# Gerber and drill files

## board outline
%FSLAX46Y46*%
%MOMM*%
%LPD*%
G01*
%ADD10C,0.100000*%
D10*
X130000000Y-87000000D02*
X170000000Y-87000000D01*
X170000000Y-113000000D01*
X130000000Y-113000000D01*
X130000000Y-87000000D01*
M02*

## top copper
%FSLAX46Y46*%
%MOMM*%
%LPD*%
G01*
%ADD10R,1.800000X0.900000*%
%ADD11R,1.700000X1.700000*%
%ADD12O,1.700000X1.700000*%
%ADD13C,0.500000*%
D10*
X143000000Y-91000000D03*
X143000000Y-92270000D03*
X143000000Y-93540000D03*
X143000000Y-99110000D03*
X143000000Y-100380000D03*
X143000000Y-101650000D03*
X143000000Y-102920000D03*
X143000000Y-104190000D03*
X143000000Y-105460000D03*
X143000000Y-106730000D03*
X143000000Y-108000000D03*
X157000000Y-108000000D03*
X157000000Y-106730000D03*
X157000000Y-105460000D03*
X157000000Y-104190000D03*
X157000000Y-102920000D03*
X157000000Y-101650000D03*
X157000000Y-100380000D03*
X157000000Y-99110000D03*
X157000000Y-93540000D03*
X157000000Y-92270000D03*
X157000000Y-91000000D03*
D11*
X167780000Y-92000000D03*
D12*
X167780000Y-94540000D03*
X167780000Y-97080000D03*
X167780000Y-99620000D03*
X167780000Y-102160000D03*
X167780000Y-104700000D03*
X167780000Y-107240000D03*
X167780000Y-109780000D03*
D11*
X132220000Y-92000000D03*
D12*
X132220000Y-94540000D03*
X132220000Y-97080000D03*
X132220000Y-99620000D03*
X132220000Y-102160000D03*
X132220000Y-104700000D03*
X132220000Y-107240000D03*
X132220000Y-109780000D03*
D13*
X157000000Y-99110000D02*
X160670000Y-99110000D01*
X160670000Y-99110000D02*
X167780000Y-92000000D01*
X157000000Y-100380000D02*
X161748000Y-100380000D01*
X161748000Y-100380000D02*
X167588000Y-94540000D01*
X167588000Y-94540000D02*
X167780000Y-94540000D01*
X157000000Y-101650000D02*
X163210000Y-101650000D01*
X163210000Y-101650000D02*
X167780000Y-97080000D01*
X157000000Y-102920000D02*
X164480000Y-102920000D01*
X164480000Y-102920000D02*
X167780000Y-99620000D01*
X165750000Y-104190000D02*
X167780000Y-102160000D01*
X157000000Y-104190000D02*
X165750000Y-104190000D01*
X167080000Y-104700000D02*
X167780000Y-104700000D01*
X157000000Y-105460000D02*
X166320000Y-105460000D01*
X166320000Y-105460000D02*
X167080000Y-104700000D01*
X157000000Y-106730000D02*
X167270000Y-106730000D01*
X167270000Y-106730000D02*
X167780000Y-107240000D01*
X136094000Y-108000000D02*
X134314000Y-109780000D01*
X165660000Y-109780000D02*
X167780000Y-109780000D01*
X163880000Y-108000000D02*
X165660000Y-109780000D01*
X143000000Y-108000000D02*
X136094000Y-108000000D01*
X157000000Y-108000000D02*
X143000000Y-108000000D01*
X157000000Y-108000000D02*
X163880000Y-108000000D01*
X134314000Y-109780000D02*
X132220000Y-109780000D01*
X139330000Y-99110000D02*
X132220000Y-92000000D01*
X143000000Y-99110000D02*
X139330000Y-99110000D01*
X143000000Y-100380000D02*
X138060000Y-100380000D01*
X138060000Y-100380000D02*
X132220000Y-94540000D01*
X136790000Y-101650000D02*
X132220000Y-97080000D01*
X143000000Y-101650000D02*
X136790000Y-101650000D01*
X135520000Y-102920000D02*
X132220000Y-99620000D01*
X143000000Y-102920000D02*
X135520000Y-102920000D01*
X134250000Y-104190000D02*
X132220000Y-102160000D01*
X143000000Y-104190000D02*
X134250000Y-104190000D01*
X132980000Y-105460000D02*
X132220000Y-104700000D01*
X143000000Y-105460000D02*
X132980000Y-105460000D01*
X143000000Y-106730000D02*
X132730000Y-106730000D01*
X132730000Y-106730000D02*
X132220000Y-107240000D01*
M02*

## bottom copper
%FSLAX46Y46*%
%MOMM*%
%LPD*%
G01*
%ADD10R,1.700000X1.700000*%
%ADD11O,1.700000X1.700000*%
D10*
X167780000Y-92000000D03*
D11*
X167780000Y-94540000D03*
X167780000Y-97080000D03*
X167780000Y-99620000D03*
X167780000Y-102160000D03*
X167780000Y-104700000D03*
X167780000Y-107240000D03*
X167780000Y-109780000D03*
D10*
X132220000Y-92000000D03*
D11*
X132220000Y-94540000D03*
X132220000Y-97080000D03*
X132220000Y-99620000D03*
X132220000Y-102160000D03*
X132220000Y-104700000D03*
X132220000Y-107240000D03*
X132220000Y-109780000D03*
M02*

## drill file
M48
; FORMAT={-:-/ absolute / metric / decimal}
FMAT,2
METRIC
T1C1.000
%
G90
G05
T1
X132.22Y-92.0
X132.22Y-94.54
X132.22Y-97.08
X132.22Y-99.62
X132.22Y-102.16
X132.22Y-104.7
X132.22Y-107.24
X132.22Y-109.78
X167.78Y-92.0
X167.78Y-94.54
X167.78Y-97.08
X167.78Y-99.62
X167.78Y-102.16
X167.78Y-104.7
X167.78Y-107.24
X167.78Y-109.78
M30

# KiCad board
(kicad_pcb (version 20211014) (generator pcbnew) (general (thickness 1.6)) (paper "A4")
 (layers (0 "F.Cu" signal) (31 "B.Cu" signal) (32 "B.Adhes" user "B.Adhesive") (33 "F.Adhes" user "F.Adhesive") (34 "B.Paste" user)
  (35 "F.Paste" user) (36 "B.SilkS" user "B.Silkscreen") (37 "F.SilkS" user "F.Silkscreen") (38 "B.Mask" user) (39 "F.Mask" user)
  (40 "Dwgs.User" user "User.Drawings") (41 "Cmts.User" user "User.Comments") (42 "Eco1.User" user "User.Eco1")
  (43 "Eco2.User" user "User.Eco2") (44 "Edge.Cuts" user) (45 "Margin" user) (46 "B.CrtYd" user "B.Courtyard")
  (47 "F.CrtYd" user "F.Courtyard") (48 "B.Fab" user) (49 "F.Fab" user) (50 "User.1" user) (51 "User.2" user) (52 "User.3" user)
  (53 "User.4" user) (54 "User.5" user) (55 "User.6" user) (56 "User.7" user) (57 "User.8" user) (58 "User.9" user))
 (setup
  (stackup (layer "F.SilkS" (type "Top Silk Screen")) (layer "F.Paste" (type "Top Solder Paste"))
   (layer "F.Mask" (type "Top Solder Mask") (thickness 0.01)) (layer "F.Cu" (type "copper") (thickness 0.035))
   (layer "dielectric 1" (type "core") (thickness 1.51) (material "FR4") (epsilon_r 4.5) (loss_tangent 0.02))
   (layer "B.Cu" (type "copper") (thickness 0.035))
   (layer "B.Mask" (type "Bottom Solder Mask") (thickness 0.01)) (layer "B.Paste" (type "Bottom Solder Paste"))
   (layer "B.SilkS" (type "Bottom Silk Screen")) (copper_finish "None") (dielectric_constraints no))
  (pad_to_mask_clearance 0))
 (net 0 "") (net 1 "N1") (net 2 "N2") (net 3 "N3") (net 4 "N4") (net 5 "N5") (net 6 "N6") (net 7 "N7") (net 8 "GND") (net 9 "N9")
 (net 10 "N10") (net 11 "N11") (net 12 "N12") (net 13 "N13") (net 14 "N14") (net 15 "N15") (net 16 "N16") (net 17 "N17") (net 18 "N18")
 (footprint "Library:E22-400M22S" (layer "F.Cu") (at 150 100)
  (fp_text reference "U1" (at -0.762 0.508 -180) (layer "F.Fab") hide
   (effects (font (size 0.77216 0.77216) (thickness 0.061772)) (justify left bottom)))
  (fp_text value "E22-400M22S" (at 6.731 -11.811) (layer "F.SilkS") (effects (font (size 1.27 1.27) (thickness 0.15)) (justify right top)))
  (pad "1" smd rect (at -7 -9 90) (size 0.9 1.8) (layers "F.Cu" "F.Paste" "F.Mask") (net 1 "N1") (solder_mask_margin 0.1016))
  (pad "2" smd rect (at -7 -7.73 90) (size 0.9 1.8) (layers "F.Cu" "F.Paste" "F.Mask") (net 1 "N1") (solder_mask_margin 0.1016))
  (pad "3" smd rect (at -7 -6.46 90) (size 0.9 1.8) (layers "F.Cu" "F.Paste" "F.Mask") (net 1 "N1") (solder_mask_margin 0.1016))
  (pad "4" smd rect (at -7 -0.89 90) (size 0.9 1.8) (layers "F.Cu" "F.Paste" "F.Mask") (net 1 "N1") (solder_mask_margin 0.1016))
  (pad "5" smd rect (at -7 0.38 90) (size 0.9 1.8) (layers "F.Cu" "F.Paste" "F.Mask") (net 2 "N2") (solder_mask_margin 0.1016))
  (pad "6" smd rect (at -7 1.65 90) (size 0.9 1.8) (layers "F.Cu" "F.Paste" "F.Mask") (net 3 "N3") (solder_mask_margin 0.1016))
  (pad "7" smd rect (at -7 2.92 90) (size 0.9 1.8) (layers "F.Cu" "F.Paste" "F.Mask") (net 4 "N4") (solder_mask_margin 0.1016))
  (pad "8" smd rect (at -7 4.19 90) (size 0.9 1.8) (layers "F.Cu" "F.Paste" "F.Mask") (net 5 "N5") (solder_mask_margin 0.1016))
  (pad "9" smd rect (at -7 5.46 90) (size 0.9 1.8) (layers "F.Cu" "F.Paste" "F.Mask") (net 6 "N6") (solder_mask_margin 0.1016))
  (pad "10" smd rect (at -7 6.73 90) (size 0.9 1.8) (layers "F.Cu" "F.Paste" "F.Mask") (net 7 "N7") (solder_mask_margin 0.1016))
  (pad "11" smd rect (at -7 8 90) (size 0.9 1.8) (layers "F.Cu" "F.Paste" "F.Mask") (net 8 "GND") (solder_mask_margin 0.1016))
  (pad "12" smd rect (at 7 8 90) (size 0.9 1.8) (layers "F.Cu" "F.Paste" "F.Mask") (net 8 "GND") (solder_mask_margin 0.1016))
  (pad "13" smd rect (at 7 6.73 90) (size 0.9 1.8) (layers "F.Cu" "F.Paste" "F.Mask") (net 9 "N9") (solder_mask_margin 0.1016))
  (pad "14" smd rect (at 7 5.46 90) (size 0.9 1.8) (layers "F.Cu" "F.Paste" "F.Mask") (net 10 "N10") (solder_mask_margin 0.1016))
  (pad "15" smd rect (at 7 4.19 90) (size 0.9 1.8) (layers "F.Cu" "F.Paste" "F.Mask") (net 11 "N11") (solder_mask_margin 0.1016))
  (pad "16" smd rect (at 7 2.92 90) (size 0.9 1.8) (layers "F.Cu" "F.Paste" "F.Mask") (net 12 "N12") (solder_mask_margin 0.1016))
  (pad "17" smd rect (at 7 1.65 90) (size 0.9 1.8) (layers "F.Cu" "F.Paste" "F.Mask") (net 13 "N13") (solder_mask_margin 0.1016))
  (pad "18" smd rect (at 7 0.38 90) (size 0.9 1.8) (layers "F.Cu" "F.Paste" "F.Mask") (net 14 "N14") (solder_mask_margin 0.1016))
  (pad "19" smd rect (at 7 -0.89 90) (size 0.9 1.8) (layers "F.Cu" "F.Paste" "F.Mask") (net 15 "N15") (solder_mask_margin 0.1016))
  (pad "20" smd rect (at 7 -6.46 90) (size 0.9 1.8) (layers "F.Cu" "F.Paste" "F.Mask") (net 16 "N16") (solder_mask_margin 0.1016))
  (pad "21" smd rect (at 7 -7.73 90) (size 0.9 1.8) (layers "F.Cu" "F.Paste" "F.Mask") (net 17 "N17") (solder_mask_margin 0.1016))
  (pad "22" smd rect (at 7 -9 90) (size 0.9 1.8) (layers "F.Cu" "F.Paste" "F.Mask") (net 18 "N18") (solder_mask_margin 0.1016)))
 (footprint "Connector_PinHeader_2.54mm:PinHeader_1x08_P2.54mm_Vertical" (layer "F.Cu") (at 167.78 92)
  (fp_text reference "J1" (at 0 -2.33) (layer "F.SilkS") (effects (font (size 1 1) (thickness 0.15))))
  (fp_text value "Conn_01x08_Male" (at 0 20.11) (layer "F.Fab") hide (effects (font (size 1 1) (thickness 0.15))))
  (pad "1" thru_hole rect (at 0 0) (size 1.7 1.7) (drill 1) (layers *.Cu *.Mask) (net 15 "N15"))
  (pad "2" thru_hole oval (at 0 2.54) (size 1.7 1.7) (drill 1) (layers *.Cu *.Mask) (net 14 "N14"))
  (pad "3" thru_hole oval (at 0 5.08) (size 1.7 1.7) (drill 1) (layers *.Cu *.Mask) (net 13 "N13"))
  (pad "4" thru_hole oval (at 0 7.62) (size 1.7 1.7) (drill 1) (layers *.Cu *.Mask) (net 12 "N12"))
  (pad "5" thru_hole oval (at 0 10.16) (size 1.7 1.7) (drill 1) (layers *.Cu *.Mask) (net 11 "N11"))
  (pad "6" thru_hole oval (at 0 12.7) (size 1.7 1.7) (drill 1) (layers *.Cu *.Mask) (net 10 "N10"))
  (pad "7" thru_hole oval (at 0 15.24) (size 1.7 1.7) (drill 1) (layers *.Cu *.Mask) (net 9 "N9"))
  (pad "8" thru_hole oval (at 0 17.78) (size 1.7 1.7) (drill 1) (layers *.Cu *.Mask) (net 8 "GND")))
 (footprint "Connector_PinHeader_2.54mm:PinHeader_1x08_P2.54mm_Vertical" (layer "F.Cu") (at 132.22 92)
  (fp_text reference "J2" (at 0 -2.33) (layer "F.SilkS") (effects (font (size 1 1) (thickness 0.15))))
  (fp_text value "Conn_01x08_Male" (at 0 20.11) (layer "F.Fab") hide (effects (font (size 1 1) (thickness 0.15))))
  (pad "1" thru_hole rect (at 0 0) (size 1.7 1.7) (drill 1) (layers *.Cu *.Mask) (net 1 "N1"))
  (pad "2" thru_hole oval (at 0 2.54) (size 1.7 1.7) (drill 1) (layers *.Cu *.Mask) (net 2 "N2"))
  (pad "3" thru_hole oval (at 0 5.08) (size 1.7 1.7) (drill 1) (layers *.Cu *.Mask) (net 3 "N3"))
  (pad "4" thru_hole oval (at 0 7.62) (size 1.7 1.7) (drill 1) (layers *.Cu *.Mask) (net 4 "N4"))
  (pad "5" thru_hole oval (at 0 10.16) (size 1.7 1.7) (drill 1) (layers *.Cu *.Mask) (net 5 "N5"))
  (pad "6" thru_hole oval (at 0 12.7) (size 1.7 1.7) (drill 1) (layers *.Cu *.Mask) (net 6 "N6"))
  (pad "7" thru_hole oval (at 0 15.24) (size 1.7 1.7) (drill 1) (layers *.Cu *.Mask) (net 7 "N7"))
  (pad "8" thru_hole oval (at 0 17.78) (size 1.7 1.7) (drill 1) (layers *.Cu *.Mask) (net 8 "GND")))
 (gr_rect (start 130 87) (end 170 113) (layer "Edge.Cuts") (width 0.1) (fill none))
 (segment (start 157 99.11) (end 160.67 99.11) (width 0.5) (layer "F.Cu") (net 15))
 (segment (start 160.67 99.11) (end 167.78 92) (width 0.5) (layer "F.Cu") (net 15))
 (segment (start 157 100.38) (end 161.748 100.38) (width 0.5) (layer "F.Cu") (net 14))
 (segment (start 161.748 100.38) (end 167.588 94.54) (width 0.5) (layer "F.Cu") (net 14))
 (segment (start 167.588 94.54) (end 167.78 94.54) (width 0.5) (layer "F.Cu") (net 14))
 (segment (start 157 101.65) (end 163.21 101.65) (width 0.5) (layer "F.Cu") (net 13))
 (segment (start 163.21 101.65) (end 167.78 97.08) (width 0.5) (layer "F.Cu") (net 13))
 (segment (start 157 102.92) (end 164.48 102.92) (width 0.5) (layer "F.Cu") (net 12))
 (segment (start 164.48 102.92) (end 167.78 99.62) (width 0.5) (layer "F.Cu") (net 12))
 (segment (start 165.75 104.19) (end 167.78 102.16) (width 0.5) (layer "F.Cu") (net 11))
 (segment (start 157 104.19) (end 165.75 104.19) (width 0.5) (layer "F.Cu") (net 11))
 (segment (start 167.08 104.7) (end 167.78 104.7) (width 0.5) (layer "F.Cu") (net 10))
 (segment (start 157 105.46) (end 166.32 105.46) (width 0.5) (layer "F.Cu") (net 10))
 (segment (start 166.32 105.46) (end 167.08 104.7) (width 0.5) (layer "F.Cu") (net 10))
 (segment (start 157 106.73) (end 167.27 106.73) (width 0.5) (layer "F.Cu") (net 9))
 (segment (start 167.27 106.73) (end 167.78 107.24) (width 0.5) (layer "F.Cu") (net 9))
 (segment (start 136.094 108) (end 134.314 109.78) (width 0.5) (layer "F.Cu") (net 8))
 (segment (start 165.66 109.78) (end 167.78 109.78) (width 0.5) (layer "F.Cu") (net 8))
 (segment (start 163.88 108) (end 165.66 109.78) (width 0.5) (layer "F.Cu") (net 8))
 (segment (start 143 108) (end 136.094 108) (width 0.5) (layer "F.Cu") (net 8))
 (segment (start 157 108) (end 143 108) (width 0.5) (layer "F.Cu") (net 8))
 (segment (start 157 108) (end 163.88 108) (width 0.5) (layer "F.Cu") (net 8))
 (segment (start 134.314 109.78) (end 132.22 109.78) (width 0.5) (layer "F.Cu") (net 8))
 (segment (start 139.33 99.11) (end 132.22 92) (width 0.5) (layer "F.Cu") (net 1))
 (segment (start 143 99.11) (end 139.33 99.11) (width 0.5) (layer "F.Cu") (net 1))
 (segment (start 143 100.38) (end 138.06 100.38) (width 0.5) (layer "F.Cu") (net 2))
 (segment (start 138.06 100.38) (end 132.22 94.54) (width 0.5) (layer "F.Cu") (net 2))
 (segment (start 136.79 101.65) (end 132.22 97.08) (width 0.5) (layer "F.Cu") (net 3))
 (segment (start 143 101.65) (end 136.79 101.65) (width 0.5) (layer "F.Cu") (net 3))
 (segment (start 135.52 102.92) (end 132.22 99.62) (width 0.5) (layer "F.Cu") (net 4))
 (segment (start 143 102.92) (end 135.52 102.92) (width 0.5) (layer "F.Cu") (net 4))
 (segment (start 134.25 104.19) (end 132.22 102.16) (width 0.5) (layer "F.Cu") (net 5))
 (segment (start 143 104.19) (end 134.25 104.19) (width 0.5) (layer "F.Cu") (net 5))
 (segment (start 132.98 105.46) (end 132.22 104.7) (width 0.5) (layer "F.Cu") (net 6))
 (segment (start 143 105.46) (end 132.98 105.46) (width 0.5) (layer "F.Cu") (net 6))
 (segment (start 143 106.73) (end 132.73 106.73) (width 0.5) (layer "F.Cu") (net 7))
 (segment (start 132.73 106.73) (end 132.22 107.24) (width 0.5) (layer "F.Cu") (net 7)))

